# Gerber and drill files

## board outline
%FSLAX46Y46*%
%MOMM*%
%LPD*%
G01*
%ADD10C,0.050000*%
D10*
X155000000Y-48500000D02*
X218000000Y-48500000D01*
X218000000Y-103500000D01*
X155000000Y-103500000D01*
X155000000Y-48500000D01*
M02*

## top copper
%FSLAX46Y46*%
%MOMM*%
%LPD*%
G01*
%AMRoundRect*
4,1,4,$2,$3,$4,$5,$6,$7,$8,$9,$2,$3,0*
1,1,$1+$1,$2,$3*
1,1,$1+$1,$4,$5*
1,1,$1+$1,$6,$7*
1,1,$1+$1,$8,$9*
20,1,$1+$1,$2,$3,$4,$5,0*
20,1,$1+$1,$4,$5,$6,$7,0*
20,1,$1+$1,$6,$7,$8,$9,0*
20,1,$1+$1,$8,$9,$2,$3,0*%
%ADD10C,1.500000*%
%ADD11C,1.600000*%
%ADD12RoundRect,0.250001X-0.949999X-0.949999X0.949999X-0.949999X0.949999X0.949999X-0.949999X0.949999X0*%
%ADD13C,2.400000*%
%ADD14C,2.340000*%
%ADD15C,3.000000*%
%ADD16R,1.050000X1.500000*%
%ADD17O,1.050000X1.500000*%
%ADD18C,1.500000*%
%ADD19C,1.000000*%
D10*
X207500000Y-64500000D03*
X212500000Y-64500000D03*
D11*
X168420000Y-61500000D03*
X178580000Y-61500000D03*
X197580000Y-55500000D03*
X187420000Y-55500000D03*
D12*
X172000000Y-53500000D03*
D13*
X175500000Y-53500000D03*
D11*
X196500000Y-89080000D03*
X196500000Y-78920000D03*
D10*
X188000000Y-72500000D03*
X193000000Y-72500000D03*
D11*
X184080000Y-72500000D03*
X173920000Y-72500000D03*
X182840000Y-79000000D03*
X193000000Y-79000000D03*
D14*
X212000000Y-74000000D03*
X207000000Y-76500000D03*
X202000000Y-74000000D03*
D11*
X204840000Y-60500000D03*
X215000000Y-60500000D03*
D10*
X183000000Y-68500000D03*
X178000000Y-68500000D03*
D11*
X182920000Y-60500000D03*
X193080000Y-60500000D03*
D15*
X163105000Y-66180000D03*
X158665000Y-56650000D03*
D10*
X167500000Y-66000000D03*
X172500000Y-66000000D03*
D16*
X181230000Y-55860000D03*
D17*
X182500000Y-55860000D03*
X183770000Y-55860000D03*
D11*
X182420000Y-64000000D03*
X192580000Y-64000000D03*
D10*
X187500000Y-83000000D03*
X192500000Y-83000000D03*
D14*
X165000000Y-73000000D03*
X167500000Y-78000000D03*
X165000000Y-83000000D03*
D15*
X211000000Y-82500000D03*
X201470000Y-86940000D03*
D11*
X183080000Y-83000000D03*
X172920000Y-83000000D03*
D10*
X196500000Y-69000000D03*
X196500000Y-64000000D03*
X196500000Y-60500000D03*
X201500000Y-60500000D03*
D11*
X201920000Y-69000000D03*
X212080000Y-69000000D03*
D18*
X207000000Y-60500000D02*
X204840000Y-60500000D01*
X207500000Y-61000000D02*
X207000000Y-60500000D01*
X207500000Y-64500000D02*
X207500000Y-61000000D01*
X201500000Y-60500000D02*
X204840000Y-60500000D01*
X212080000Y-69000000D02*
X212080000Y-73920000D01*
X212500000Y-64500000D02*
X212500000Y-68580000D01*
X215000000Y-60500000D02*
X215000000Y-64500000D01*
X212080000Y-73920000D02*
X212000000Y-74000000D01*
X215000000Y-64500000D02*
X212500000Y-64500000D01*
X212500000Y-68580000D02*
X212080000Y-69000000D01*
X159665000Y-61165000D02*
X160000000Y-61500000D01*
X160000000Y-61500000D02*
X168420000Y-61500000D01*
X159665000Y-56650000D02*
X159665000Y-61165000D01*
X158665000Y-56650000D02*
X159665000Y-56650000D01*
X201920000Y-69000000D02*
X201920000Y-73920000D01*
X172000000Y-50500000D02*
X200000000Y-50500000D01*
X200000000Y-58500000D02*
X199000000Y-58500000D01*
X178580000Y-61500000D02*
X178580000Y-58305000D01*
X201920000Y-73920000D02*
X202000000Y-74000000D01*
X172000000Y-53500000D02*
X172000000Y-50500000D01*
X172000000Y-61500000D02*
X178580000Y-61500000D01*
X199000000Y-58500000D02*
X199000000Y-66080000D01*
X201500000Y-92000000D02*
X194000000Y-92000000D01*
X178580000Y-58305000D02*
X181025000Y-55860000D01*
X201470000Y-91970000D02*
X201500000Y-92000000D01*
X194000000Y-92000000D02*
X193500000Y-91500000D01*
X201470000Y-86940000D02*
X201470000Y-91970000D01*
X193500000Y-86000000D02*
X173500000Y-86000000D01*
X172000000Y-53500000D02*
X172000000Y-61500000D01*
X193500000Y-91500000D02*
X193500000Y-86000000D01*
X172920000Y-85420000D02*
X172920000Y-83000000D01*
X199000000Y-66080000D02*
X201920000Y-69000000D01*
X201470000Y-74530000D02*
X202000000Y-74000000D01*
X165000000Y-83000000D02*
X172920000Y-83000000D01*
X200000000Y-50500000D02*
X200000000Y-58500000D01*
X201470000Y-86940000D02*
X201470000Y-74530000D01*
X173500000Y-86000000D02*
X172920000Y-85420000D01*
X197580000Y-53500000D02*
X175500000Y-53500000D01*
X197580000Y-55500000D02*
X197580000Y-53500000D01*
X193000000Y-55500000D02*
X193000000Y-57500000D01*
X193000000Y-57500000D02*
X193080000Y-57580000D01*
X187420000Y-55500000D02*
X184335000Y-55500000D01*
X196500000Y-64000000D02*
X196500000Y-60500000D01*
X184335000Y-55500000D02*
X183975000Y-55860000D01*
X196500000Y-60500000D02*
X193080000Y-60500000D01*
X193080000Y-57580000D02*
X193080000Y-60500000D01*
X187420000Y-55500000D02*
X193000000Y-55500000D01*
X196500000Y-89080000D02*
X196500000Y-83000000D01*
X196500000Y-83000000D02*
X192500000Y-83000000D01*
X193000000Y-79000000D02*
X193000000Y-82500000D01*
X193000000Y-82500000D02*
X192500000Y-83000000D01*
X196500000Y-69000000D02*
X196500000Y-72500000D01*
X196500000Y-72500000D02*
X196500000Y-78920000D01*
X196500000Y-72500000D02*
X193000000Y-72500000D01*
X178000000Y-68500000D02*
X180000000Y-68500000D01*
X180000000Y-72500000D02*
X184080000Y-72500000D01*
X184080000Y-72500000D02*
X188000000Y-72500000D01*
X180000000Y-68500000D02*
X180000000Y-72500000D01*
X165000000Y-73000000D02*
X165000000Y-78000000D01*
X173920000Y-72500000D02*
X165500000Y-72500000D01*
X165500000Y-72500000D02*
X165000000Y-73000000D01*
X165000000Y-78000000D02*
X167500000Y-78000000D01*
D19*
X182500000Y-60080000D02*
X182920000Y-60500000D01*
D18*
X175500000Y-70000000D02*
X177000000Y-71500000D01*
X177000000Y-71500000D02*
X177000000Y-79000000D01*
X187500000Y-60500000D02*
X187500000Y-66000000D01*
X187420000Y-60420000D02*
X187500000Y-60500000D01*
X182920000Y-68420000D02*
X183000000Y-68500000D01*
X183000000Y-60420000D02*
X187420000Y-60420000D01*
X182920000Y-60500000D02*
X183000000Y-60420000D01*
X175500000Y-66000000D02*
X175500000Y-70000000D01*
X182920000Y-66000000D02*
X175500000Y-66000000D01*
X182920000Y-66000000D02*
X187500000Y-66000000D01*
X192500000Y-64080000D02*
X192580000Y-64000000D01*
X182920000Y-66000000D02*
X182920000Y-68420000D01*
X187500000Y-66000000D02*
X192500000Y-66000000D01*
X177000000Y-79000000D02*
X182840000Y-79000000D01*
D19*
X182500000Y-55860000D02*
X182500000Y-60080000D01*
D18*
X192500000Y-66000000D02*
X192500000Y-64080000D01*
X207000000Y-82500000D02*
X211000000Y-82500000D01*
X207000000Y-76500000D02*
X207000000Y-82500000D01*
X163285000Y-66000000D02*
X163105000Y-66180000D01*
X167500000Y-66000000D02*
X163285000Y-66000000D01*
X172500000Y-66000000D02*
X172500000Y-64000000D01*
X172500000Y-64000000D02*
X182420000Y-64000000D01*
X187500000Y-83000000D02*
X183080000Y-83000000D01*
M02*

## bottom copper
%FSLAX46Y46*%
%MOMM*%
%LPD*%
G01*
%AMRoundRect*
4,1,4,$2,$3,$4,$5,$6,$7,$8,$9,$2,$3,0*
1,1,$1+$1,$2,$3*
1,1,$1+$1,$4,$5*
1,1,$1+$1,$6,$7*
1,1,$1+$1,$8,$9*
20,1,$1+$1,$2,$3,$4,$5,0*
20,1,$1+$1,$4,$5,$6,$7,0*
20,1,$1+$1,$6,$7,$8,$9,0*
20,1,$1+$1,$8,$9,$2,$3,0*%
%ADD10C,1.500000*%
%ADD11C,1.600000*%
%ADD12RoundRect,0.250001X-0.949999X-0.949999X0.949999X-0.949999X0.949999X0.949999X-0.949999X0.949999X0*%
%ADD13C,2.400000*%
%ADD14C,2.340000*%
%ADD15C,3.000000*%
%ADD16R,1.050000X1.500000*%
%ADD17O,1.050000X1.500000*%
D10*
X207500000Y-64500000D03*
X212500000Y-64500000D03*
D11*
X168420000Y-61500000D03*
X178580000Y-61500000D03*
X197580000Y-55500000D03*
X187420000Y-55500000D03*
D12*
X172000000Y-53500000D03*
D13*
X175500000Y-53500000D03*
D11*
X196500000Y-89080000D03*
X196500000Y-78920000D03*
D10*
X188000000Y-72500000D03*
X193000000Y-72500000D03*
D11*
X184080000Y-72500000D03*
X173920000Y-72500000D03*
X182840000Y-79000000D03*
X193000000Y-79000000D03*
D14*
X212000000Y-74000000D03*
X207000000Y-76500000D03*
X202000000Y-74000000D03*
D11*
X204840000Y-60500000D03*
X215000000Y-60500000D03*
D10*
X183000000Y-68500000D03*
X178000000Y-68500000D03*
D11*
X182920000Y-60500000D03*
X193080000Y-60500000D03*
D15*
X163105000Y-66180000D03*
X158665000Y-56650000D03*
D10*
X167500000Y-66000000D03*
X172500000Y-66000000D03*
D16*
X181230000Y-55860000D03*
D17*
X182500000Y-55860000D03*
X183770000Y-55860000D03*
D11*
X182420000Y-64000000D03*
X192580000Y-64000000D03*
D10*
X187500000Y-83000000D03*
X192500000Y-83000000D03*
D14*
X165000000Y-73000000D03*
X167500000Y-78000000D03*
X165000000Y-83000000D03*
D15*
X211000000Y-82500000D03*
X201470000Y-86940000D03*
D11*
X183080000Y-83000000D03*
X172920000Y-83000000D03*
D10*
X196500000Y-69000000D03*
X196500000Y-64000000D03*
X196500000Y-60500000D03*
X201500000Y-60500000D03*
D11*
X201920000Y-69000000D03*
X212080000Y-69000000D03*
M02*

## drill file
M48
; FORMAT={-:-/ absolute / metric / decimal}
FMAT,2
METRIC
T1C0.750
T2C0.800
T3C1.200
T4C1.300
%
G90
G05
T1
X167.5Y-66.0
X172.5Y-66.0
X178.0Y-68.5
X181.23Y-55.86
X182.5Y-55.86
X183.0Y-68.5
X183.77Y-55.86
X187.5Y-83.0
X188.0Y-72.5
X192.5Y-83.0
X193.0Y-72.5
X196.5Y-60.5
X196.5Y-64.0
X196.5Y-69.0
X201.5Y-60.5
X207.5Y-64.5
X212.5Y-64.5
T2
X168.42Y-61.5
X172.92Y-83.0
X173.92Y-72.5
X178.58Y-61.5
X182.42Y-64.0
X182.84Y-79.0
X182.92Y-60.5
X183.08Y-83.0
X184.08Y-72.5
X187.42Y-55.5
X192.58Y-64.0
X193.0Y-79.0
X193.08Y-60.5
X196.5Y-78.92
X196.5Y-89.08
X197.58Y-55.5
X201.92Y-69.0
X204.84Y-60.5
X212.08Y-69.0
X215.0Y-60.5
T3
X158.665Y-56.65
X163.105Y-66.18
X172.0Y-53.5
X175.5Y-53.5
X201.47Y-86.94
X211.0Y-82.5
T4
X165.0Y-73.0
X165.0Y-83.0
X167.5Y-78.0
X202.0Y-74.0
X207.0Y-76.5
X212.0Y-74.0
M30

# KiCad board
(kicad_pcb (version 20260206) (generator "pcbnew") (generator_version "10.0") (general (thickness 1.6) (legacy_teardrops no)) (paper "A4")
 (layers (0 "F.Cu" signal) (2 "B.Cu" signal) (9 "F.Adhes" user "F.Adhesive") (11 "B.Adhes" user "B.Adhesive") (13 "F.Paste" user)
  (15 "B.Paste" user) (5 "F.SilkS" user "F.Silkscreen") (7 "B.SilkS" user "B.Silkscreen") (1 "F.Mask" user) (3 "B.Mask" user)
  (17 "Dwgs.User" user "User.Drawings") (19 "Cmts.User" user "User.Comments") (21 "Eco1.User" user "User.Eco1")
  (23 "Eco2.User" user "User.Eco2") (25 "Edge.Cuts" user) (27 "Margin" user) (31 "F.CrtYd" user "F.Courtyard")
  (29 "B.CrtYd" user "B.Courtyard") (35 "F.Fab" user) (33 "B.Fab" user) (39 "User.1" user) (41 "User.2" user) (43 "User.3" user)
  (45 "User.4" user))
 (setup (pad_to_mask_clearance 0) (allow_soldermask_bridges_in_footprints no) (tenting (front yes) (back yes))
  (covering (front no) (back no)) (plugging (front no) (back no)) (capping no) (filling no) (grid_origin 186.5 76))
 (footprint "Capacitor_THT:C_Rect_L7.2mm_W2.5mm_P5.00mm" (layer "F.Cu") (at 207.5 64.5)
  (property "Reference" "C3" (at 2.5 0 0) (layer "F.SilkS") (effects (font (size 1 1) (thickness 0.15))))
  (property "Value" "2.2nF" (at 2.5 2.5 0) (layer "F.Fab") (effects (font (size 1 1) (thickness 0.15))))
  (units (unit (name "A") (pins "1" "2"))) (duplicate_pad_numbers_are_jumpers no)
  (pad "1" thru_hole circle (at 0 0) (size 1.5 1.5) (drill 0.75) (layers "*.Cu" "*.Mask") (remove_unused_layers no) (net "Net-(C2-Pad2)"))
  (pad "2" thru_hole circle (at 5 0) (size 1.5 1.5) (drill 0.75) (layers "*.Cu" "*.Mask") (remove_unused_layers no) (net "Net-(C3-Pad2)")))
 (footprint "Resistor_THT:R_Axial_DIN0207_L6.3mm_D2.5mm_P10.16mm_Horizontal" (layer "F.Cu") (at 168.42 61.5)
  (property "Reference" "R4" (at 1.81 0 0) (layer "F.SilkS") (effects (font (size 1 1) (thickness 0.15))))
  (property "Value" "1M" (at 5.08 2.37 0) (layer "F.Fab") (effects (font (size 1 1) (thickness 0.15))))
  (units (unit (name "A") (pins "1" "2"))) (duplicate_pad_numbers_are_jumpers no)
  (pad "1" thru_hole circle (at 0 0) (size 1.6 1.6) (drill 0.8) (layers "*.Cu" "*.Mask") (remove_unused_layers no) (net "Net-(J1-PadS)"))
  (pad "2" thru_hole circle (at 10.16 0) (size 1.6 1.6) (drill 0.8) (layers "*.Cu" "*.Mask") (remove_unused_layers no) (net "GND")))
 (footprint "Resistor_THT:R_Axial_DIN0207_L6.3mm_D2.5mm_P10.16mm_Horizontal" (layer "F.Cu") (at 197.58 55.5 180)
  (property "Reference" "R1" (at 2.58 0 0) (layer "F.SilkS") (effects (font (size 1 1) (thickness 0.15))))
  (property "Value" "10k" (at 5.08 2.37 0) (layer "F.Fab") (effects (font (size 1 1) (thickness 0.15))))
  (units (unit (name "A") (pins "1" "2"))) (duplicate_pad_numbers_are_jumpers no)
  (pad "1" thru_hole circle (at 0 0 180) (size 1.6 1.6) (drill 0.8) (layers "*.Cu" "*.Mask") (remove_unused_layers no) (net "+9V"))
  (pad "2" thru_hole circle (at 10.16 0 180) (size 1.6 1.6) (drill 0.8) (layers "*.Cu" "*.Mask") (remove_unused_layers no)
   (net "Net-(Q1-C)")))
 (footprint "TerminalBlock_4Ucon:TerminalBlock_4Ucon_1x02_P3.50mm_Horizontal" (layer "F.Cu") (at 172 53.5)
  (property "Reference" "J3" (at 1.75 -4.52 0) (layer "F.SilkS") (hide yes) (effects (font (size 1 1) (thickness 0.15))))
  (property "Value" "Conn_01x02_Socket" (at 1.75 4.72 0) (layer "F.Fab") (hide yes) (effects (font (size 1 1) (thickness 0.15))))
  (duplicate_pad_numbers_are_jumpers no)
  (pad "1" thru_hole roundrect (at 0 0) (size 2.4 2.4) (drill 1.2) (layers "*.Cu" "*.Mask") (remove_unused_layers no)
   (roundrect_rratio 0.104167) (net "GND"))
  (pad "2" thru_hole circle (at 3.5 0) (size 2.4 2.4) (drill 1.2) (layers "*.Cu" "*.Mask") (remove_unused_layers no) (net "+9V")))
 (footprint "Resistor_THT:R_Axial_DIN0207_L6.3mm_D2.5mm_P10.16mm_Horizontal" (layer "F.Cu") (at 196.5 89.08 90)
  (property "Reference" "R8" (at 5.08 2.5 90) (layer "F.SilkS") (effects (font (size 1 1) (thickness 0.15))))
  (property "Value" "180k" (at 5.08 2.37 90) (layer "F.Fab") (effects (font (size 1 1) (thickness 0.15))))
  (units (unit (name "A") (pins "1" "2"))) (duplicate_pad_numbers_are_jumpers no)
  (pad "1" thru_hole circle (at 0 0 90) (size 1.6 1.6) (drill 0.8) (layers "*.Cu" "*.Mask") (remove_unused_layers no) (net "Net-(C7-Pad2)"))
  (pad "2" thru_hole circle (at 10.16 0 90) (size 1.6 1.6) (drill 0.8) (layers "*.Cu" "*.Mask") (remove_unused_layers no)
   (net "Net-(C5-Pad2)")))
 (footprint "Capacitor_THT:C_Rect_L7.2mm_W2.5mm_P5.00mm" (layer "F.Cu") (at 188 72.5)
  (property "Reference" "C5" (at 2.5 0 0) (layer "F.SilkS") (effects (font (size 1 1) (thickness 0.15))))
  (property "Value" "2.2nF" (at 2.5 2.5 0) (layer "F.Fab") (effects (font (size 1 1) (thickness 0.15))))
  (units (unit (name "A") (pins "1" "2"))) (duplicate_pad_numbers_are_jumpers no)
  (pad "1" thru_hole circle (at 0 0) (size 1.5 1.5) (drill 0.75) (layers "*.Cu" "*.Mask") (remove_unused_layers no) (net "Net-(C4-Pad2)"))
  (pad "2" thru_hole circle (at 5 0) (size 1.5 1.5) (drill 0.75) (layers "*.Cu" "*.Mask") (remove_unused_layers no) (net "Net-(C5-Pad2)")))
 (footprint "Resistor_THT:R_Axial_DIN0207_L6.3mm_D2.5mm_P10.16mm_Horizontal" (layer "F.Cu") (at 184.08 72.5 180)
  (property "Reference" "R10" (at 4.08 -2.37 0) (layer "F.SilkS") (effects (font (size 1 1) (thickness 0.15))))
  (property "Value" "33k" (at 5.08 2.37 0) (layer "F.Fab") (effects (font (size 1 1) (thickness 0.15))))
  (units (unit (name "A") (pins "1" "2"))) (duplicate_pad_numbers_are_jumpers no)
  (pad "1" thru_hole circle (at 0 0 180) (size 1.6 1.6) (drill 0.8) (layers "*.Cu" "*.Mask") (remove_unused_layers no) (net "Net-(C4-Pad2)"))
  (pad "2" thru_hole circle (at 10.16 0 180) (size 1.6 1.6) (drill 0.8) (layers "*.Cu" "*.Mask") (remove_unused_layers no)
   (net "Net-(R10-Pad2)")))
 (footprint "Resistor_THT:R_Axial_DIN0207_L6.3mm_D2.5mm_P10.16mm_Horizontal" (layer "F.Cu") (at 182.84 79)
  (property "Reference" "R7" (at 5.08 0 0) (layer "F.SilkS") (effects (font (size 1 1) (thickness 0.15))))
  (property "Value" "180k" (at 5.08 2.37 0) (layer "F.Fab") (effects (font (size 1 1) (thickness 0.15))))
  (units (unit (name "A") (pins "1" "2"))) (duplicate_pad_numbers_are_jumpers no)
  (pad "1" thru_hole circle (at 0 0) (size 1.6 1.6) (drill 0.8) (layers "*.Cu" "*.Mask") (remove_unused_layers no) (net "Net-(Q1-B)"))
  (pad "2" thru_hole circle (at 10.16 0) (size 1.6 1.6) (drill 0.8) (layers "*.Cu" "*.Mask") (remove_unused_layers no) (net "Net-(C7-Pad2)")))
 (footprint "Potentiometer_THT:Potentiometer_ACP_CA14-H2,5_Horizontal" (layer "F.Cu") (at 212 74 -90)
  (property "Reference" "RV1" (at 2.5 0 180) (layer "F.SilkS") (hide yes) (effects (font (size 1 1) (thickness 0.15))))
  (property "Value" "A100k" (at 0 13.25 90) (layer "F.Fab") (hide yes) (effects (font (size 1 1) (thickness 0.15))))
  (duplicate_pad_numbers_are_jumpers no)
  (pad "1" thru_hole circle (at 0 0 270) (size 2.34 2.34) (drill 1.3) (layers "*.Cu" "*.Mask") (remove_unused_layers no)
   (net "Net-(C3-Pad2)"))
  (pad "2" thru_hole circle (at 2.5 5 270) (size 2.34 2.34) (drill 1.3) (layers "*.Cu" "*.Mask") (remove_unused_layers no)
   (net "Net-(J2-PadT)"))
  (pad "3" thru_hole circle (at 0 10 270) (size 2.34 2.34) (drill 1.3) (layers "*.Cu" "*.Mask") (remove_unused_layers no) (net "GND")))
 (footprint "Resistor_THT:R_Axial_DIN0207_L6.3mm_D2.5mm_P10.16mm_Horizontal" (layer "F.Cu") (at 204.84 60.5)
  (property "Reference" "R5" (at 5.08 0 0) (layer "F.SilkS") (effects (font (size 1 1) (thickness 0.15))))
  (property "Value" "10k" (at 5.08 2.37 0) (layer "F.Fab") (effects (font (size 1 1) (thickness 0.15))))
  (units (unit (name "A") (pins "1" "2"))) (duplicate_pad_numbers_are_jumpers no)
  (pad "1" thru_hole circle (at 0 0) (size 1.6 1.6) (drill 0.8) (layers "*.Cu" "*.Mask") (remove_unused_layers no) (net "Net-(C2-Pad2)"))
  (pad "2" thru_hole circle (at 10.16 0) (size 1.6 1.6) (drill 0.8) (layers "*.Cu" "*.Mask") (remove_unused_layers no) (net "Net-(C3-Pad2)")))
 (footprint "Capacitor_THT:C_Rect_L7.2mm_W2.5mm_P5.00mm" (layer "F.Cu") (at 183 68.5 180)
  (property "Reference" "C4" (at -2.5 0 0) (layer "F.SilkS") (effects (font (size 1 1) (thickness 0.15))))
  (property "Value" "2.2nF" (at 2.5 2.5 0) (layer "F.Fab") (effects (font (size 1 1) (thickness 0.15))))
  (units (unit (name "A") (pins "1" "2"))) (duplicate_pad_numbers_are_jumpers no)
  (pad "1" thru_hole circle (at 0 0 180) (size 1.5 1.5) (drill 0.75) (layers "*.Cu" "*.Mask") (remove_unused_layers no) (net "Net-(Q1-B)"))
  (pad "2" thru_hole circle (at 5 0 180) (size 1.5 1.5) (drill 0.75) (layers "*.Cu" "*.Mask") (remove_unused_layers no)
   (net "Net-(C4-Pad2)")))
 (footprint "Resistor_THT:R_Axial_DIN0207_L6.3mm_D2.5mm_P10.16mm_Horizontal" (layer "F.Cu") (at 182.92 60.5)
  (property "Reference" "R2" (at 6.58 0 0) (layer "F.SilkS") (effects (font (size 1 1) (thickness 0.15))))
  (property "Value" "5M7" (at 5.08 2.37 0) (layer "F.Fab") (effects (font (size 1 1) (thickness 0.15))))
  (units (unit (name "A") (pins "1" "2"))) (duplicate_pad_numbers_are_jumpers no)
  (pad "1" thru_hole circle (at 0 0) (size 1.6 1.6) (drill 0.8) (layers "*.Cu" "*.Mask") (remove_unused_layers no) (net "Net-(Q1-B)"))
  (pad "2" thru_hole circle (at 10.16 0) (size 1.6 1.6) (drill 0.8) (layers "*.Cu" "*.Mask") (remove_unused_layers no) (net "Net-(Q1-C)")))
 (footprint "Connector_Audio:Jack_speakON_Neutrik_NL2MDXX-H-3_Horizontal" (layer "F.Cu") (at 163.105 66.18 180)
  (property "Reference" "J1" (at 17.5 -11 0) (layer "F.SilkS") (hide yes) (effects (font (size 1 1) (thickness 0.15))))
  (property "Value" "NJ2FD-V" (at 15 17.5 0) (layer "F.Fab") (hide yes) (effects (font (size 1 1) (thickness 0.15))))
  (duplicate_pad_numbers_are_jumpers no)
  (pad "1+" thru_hole circle (at 0 0 180) (size 3 3) (drill 1.2) (layers "*.Cu" "*.Mask") (remove_unused_layers no) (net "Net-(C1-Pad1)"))
  (pad "1-" thru_hole circle (at 4.44 9.53 180) (size 3 3) (drill 1.2) (layers "*.Cu" "*.Mask") (remove_unused_layers no)
   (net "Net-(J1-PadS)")))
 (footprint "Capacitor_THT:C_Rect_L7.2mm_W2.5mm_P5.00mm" (layer "F.Cu") (at 167.5 66)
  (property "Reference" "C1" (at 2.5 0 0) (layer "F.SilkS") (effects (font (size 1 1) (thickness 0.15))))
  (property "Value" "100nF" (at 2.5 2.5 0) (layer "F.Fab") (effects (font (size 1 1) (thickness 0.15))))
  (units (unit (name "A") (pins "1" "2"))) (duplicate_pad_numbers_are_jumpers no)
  (pad "1" thru_hole circle (at 0 0) (size 1.5 1.5) (drill 0.75) (layers "*.Cu" "*.Mask") (remove_unused_layers no) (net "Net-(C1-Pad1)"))
  (pad "2" thru_hole circle (at 5 0) (size 1.5 1.5) (drill 0.75) (layers "*.Cu" "*.Mask") (remove_unused_layers no) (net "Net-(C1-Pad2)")))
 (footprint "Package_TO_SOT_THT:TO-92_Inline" (layer "F.Cu") (at 181.23 55.86)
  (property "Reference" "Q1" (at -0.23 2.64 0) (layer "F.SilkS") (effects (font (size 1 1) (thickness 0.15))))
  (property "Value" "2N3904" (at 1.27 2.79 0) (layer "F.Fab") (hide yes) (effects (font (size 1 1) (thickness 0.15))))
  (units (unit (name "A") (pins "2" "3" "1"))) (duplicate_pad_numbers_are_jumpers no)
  (pad "1" thru_hole rect (at 0 0) (size 1.05 1.5) (drill 0.75) (layers "*.Cu" "*.Mask") (remove_unused_layers no) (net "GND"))
  (pad "2" thru_hole oval (at 1.27 0) (size 1.05 1.5) (drill 0.75) (layers "*.Cu" "*.Mask") (remove_unused_layers no) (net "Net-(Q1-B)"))
  (pad "3" thru_hole oval (at 2.54 0) (size 1.05 1.5) (drill 0.75) (layers "*.Cu" "*.Mask") (remove_unused_layers no) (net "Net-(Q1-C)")))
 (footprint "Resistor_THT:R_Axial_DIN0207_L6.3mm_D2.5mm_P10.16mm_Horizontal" (layer "F.Cu") (at 182.42 64)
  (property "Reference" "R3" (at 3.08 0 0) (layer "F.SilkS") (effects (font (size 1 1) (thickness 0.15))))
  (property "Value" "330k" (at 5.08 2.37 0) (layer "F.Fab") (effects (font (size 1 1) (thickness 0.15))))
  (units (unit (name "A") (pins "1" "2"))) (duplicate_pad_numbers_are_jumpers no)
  (pad "1" thru_hole circle (at 0 0) (size 1.6 1.6) (drill 0.8) (layers "*.Cu" "*.Mask") (remove_unused_layers no) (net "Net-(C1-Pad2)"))
  (pad "2" thru_hole circle (at 10.16 0) (size 1.6 1.6) (drill 0.8) (layers "*.Cu" "*.Mask") (remove_unused_layers no) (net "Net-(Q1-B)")))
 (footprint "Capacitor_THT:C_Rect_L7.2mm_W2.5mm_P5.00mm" (layer "F.Cu") (at 187.5 83)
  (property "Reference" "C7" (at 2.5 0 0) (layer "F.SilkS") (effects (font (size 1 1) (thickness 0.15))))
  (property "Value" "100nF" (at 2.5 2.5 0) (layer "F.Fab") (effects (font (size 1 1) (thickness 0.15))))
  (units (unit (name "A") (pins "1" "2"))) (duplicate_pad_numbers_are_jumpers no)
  (pad "1" thru_hole circle (at 0 0) (size 1.5 1.5) (drill 0.75) (layers "*.Cu" "*.Mask") (remove_unused_layers no) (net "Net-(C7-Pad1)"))
  (pad "2" thru_hole circle (at 5 0) (size 1.5 1.5) (drill 0.75) (layers "*.Cu" "*.Mask") (remove_unused_layers no) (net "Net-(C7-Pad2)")))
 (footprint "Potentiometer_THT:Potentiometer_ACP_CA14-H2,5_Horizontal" (layer "F.Cu") (at 165 73)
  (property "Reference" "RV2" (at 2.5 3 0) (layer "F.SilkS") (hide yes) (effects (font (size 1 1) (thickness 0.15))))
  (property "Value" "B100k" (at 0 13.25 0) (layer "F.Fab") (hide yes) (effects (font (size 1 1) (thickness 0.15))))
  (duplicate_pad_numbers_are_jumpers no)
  (pad "1" thru_hole circle (at 0 0) (size 2.34 2.34) (drill 1.3) (layers "*.Cu" "*.Mask") (remove_unused_layers no) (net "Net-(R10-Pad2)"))
  (pad "2" thru_hole circle (at 2.5 5) (size 2.34 2.34) (drill 1.3) (layers "*.Cu" "*.Mask") (remove_unused_layers no)
   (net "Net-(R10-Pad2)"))
  (pad "3" thru_hole circle (at 0 10) (size 2.34 2.34) (drill 1.3) (layers "*.Cu" "*.Mask") (remove_unused_layers no) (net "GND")))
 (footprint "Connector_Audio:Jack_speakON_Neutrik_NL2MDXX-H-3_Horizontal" (layer "F.Cu") (at 211 82.5 -90)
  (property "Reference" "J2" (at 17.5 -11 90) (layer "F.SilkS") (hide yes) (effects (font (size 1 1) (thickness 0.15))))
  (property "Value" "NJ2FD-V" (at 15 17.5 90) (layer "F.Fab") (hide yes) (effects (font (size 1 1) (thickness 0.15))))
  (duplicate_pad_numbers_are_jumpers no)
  (pad "1+" thru_hole circle (at 0 0 270) (size 3 3) (drill 1.2) (layers "*.Cu" "*.Mask") (remove_unused_layers no) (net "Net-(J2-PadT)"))
  (pad "1-" thru_hole circle (at 4.44 9.53 270) (size 3 3) (drill 1.2) (layers "*.Cu" "*.Mask") (remove_unused_layers no) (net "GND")))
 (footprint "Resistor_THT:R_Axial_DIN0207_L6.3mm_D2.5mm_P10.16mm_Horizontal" (layer "F.Cu") (at 183.08 83 180)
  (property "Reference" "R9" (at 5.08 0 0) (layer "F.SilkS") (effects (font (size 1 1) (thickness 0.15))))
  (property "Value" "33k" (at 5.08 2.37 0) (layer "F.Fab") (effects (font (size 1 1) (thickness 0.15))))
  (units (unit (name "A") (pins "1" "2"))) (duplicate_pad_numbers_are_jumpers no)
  (pad "1" thru_hole circle (at 0 0 180) (size 1.6 1.6) (drill 0.8) (layers "*.Cu" "*.Mask") (remove_unused_layers no) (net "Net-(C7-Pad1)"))
  (pad "2" thru_hole circle (at 10.16 0 180) (size 1.6 1.6) (drill 0.8) (layers "*.Cu" "*.Mask") (remove_unused_layers no) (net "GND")))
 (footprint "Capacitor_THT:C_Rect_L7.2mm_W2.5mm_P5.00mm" (layer "F.Cu") (at 196.5 69 90)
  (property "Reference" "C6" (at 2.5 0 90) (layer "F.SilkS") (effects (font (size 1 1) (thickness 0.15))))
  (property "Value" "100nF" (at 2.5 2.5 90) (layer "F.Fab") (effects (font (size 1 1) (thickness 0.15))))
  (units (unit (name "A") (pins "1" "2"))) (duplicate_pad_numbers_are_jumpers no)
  (pad "1" thru_hole circle (at 0 0 90) (size 1.5 1.5) (drill 0.75) (layers "*.Cu" "*.Mask") (remove_unused_layers no) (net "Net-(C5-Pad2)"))
  (pad "2" thru_hole circle (at 5 0 90) (size 1.5 1.5) (drill 0.75) (layers "*.Cu" "*.Mask") (remove_unused_layers no) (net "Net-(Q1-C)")))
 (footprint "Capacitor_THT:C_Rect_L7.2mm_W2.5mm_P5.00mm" (layer "F.Cu") (at 196.5 60.5)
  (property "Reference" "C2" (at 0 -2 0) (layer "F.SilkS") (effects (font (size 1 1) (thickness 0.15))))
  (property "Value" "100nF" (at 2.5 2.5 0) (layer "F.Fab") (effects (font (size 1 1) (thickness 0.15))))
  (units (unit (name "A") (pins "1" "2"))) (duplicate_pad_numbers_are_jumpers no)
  (pad "1" thru_hole circle (at 0 0) (size 1.5 1.5) (drill 0.75) (layers "*.Cu" "*.Mask") (remove_unused_layers no) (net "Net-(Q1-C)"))
  (pad "2" thru_hole circle (at 5 0) (size 1.5 1.5) (drill 0.75) (layers "*.Cu" "*.Mask") (remove_unused_layers no) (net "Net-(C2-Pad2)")))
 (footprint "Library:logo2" (layer "F.Cu") (at 186.500278 97.619189)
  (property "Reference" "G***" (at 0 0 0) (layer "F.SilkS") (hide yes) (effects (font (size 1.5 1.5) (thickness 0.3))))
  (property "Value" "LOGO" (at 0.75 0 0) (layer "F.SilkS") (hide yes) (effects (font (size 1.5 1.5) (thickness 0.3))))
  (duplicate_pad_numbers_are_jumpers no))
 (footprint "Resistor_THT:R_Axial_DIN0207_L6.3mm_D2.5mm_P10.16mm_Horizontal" (layer "F.Cu") (at 201.92 69)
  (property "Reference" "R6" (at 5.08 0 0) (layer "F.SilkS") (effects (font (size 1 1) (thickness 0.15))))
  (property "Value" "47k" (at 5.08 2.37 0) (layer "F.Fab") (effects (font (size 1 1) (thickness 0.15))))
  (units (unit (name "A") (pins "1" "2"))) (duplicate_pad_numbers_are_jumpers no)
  (pad "1" thru_hole circle (at 0 0) (size 1.6 1.6) (drill 0.8) (layers "*.Cu" "*.Mask") (remove_unused_layers no) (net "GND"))
  (pad "2" thru_hole circle (at 10.16 0) (size 1.6 1.6) (drill 0.8) (layers "*.Cu" "*.Mask") (remove_unused_layers no) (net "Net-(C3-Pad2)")))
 (gr_rect (start 155 48.5) (end 218 103.5) (stroke (width 0.05) (type default)) (fill no) (layer "Edge.Cuts"))
 (segment (start 207 60.5) (end 204.84 60.5) (width 1.5) (layer "F.Cu") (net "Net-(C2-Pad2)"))
 (segment (start 207.5 61) (end 207 60.5) (width 1.5) (layer "F.Cu") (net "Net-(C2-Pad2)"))
 (segment (start 207.5 64.5) (end 207.5 61) (width 1.5) (layer "F.Cu") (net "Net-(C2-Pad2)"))
 (segment (start 201.5 60.5) (end 204.84 60.5) (width 1.5) (layer "F.Cu") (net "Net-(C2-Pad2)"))
 (segment (start 212.08 69) (end 212.08 73.92) (width 1.5) (layer "F.Cu") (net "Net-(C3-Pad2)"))
 (segment (start 212.5 64.5) (end 212.5 68.58) (width 1.5) (layer "F.Cu") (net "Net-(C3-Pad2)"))
 (segment (start 215 60.5) (end 215 64.5) (width 1.5) (layer "F.Cu") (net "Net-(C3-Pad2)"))
 (segment (start 212.08 73.92) (end 212 74) (width 1.5) (layer "F.Cu") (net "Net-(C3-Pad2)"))
 (segment (start 215 64.5) (end 212.5 64.5) (width 1.5) (layer "F.Cu") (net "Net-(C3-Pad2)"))
 (segment (start 212.5 68.58) (end 212.08 69) (width 1.5) (layer "F.Cu") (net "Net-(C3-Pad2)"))
 (segment (start 159.665 61.165) (end 160 61.5) (width 1.5) (layer "F.Cu") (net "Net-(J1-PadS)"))
 (segment (start 160 61.5) (end 168.42 61.5) (width 1.5) (layer "F.Cu") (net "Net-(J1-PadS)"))
 (segment (start 159.665 56.65) (end 159.665 61.165) (width 1.5) (layer "F.Cu") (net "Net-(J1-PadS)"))
 (segment (start 158.665 56.65) (end 159.665 56.65) (width 1.5) (layer "F.Cu") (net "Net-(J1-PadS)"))
 (segment (start 201.92 69) (end 201.92 73.92) (width 1.5) (layer "F.Cu") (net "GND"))
 (segment (start 172 50.5) (end 200 50.5) (width 1.5) (layer "F.Cu") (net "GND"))
 (segment (start 200 58.5) (end 199 58.5) (width 1.5) (layer "F.Cu") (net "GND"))
 (segment (start 178.58 61.5) (end 178.58 58.305) (width 1.5) (layer "F.Cu") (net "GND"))
 (segment (start 201.92 73.92) (end 202 74) (width 1.5) (layer "F.Cu") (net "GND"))
 (segment (start 172 53.5) (end 172 50.5) (width 1.5) (layer "F.Cu") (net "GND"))
 (segment (start 172 61.5) (end 178.58 61.5) (width 1.5) (layer "F.Cu") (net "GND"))
 (segment (start 199 58.5) (end 199 66.08) (width 1.5) (layer "F.Cu") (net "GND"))
 (segment (start 201.5 92) (end 194 92) (width 1.5) (layer "F.Cu") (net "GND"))
 (segment (start 178.58 58.305) (end 181.025 55.86) (width 1.5) (layer "F.Cu") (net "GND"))
 (segment (start 201.47 91.97) (end 201.5 92) (width 1.5) (layer "F.Cu") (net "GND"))
 (segment (start 194 92) (end 193.5 91.5) (width 1.5) (layer "F.Cu") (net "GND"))
 (segment (start 201.47 86.94) (end 201.47 91.97) (width 1.5) (layer "F.Cu") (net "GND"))
 (segment (start 193.5 86) (end 173.5 86) (width 1.5) (layer "F.Cu") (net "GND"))
 (segment (start 172 53.5) (end 172 61.5) (width 1.5) (layer "F.Cu") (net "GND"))
 (segment (start 193.5 91.5) (end 193.5 86) (width 1.5) (layer "F.Cu") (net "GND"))
 (segment (start 172.92 85.42) (end 172.92 83) (width 1.5) (layer "F.Cu") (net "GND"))
 (segment (start 199 66.08) (end 201.92 69) (width 1.5) (layer "F.Cu") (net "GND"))
 (segment (start 201.47 74.53) (end 202 74) (width 1.5) (layer "F.Cu") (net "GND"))
 (segment (start 165 83) (end 172.92 83) (width 1.5) (layer "F.Cu") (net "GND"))
 (segment (start 200 50.5) (end 200 58.5) (width 1.5) (layer "F.Cu") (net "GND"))
 (segment (start 201.47 86.94) (end 201.47 74.53) (width 1.5) (layer "F.Cu") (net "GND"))
 (segment (start 173.5 86) (end 172.92 85.42) (width 1.5) (layer "F.Cu") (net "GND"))
 (segment (start 197.58 53.5) (end 175.5 53.5) (width 1.5) (layer "F.Cu") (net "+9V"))
 (segment (start 197.58 55.5) (end 197.58 53.5) (width 1.5) (layer "F.Cu") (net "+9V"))
 (segment (start 193 55.5) (end 193 57.5) (width 1.5) (layer "F.Cu") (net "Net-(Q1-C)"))
 (segment (start 193 57.5) (end 193.08 57.58) (width 1.5) (layer "F.Cu") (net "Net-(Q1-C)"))
 (segment (start 187.42 55.5) (end 184.335 55.5) (width 1.5) (layer "F.Cu") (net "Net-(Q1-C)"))
 (segment (start 196.5 64) (end 196.5 60.5) (width 1.5) (layer "F.Cu") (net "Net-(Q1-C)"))
 (segment (start 184.335 55.5) (end 183.975 55.86) (width 1.5) (layer "F.Cu") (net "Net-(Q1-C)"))
 (segment (start 196.5 60.5) (end 193.08 60.5) (width 1.5) (layer "F.Cu") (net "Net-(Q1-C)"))
 (segment (start 193.08 57.58) (end 193.08 60.5) (width 1.5) (layer "F.Cu") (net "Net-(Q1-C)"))
 (segment (start 187.42 55.5) (end 193 55.5) (width 1.5) (layer "F.Cu") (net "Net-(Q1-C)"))
 (segment (start 196.5 89.08) (end 196.5 83) (width 1.5) (layer "F.Cu") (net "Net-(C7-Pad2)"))
 (segment (start 196.5 83) (end 192.5 83) (width 1.5) (layer "F.Cu") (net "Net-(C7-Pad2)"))
 (segment (start 193 79) (end 193 82.5) (width 1.5) (layer "F.Cu") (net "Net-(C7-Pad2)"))
 (segment (start 193 82.5) (end 192.5 83) (width 1.5) (layer "F.Cu") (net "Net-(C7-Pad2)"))
 (segment (start 196.5 69) (end 196.5 72.5) (width 1.5) (layer "F.Cu") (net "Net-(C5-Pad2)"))
 (segment (start 196.5 72.5) (end 196.5 78.92) (width 1.5) (layer "F.Cu") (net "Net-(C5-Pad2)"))
 (segment (start 196.5 72.5) (end 193 72.5) (width 1.5) (layer "F.Cu") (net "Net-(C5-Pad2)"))
 (segment (start 178 68.5) (end 180 68.5) (width 1.5) (layer "F.Cu") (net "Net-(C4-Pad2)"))
 (segment (start 180 72.5) (end 184.08 72.5) (width 1.5) (layer "F.Cu") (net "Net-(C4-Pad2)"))
 (segment (start 184.08 72.5) (end 188 72.5) (width 1.5) (layer "F.Cu") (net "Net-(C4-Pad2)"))
 (segment (start 180 68.5) (end 180 72.5) (width 1.5) (layer "F.Cu") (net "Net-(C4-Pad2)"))
 (segment (start 165 73) (end 165 78) (width 1.5) (layer "F.Cu") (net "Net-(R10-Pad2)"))
 (segment (start 173.92 72.5) (end 165.5 72.5) (width 1.5) (layer "F.Cu") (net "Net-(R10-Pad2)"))
 (segment (start 165.5 72.5) (end 165 73) (width 1.5) (layer "F.Cu") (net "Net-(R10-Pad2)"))
 (segment (start 165 78) (end 167.5 78) (width 1.5) (layer "F.Cu") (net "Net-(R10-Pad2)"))
 (segment (start 182.5 60.08) (end 182.92 60.5) (width 1) (layer "F.Cu") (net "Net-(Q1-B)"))
 (segment (start 175.5 70) (end 177 71.5) (width 1.5) (layer "F.Cu") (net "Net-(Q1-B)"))
 (segment (start 177 71.5) (end 177 79) (width 1.5) (layer "F.Cu") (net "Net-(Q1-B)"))
 (segment (start 187.5 60.5) (end 187.5 66) (width 1.5) (layer "F.Cu") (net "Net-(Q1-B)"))
 (segment (start 187.42 60.42) (end 187.5 60.5) (width 1.5) (layer "F.Cu") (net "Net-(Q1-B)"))
 (segment (start 182.92 68.42) (end 183 68.5) (width 1.5) (layer "F.Cu") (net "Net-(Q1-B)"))
 (segment (start 183 60.42) (end 187.42 60.42) (width 1.5) (layer "F.Cu") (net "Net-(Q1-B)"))
 (segment (start 182.92 60.5) (end 183 60.42) (width 1.5) (layer "F.Cu") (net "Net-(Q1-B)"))
 (segment (start 175.5 66) (end 175.5 70) (width 1.5) (layer "F.Cu") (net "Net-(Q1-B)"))
 (segment (start 182.92 66) (end 175.5 66) (width 1.5) (layer "F.Cu") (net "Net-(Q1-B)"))
 (segment (start 182.92 66) (end 187.5 66) (width 1.5) (layer "F.Cu") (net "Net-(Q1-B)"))
 (segment (start 192.5 64.08) (end 192.58 64) (width 1.5) (layer "F.Cu") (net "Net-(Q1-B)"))
 (segment (start 182.92 66) (end 182.92 68.42) (width 1.5) (layer "F.Cu") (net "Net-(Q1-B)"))
 (segment (start 187.5 66) (end 192.5 66) (width 1.5) (layer "F.Cu") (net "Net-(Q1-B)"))
 (segment (start 177 79) (end 182.84 79) (width 1.5) (layer "F.Cu") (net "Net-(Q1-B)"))
 (segment (start 182.5 55.86) (end 182.5 60.08) (width 1) (layer "F.Cu") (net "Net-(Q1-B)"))
 (segment (start 192.5 66) (end 192.5 64.08) (width 1.5) (layer "F.Cu") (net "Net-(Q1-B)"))
 (segment (start 207 82.5) (end 211 82.5) (width 1.5) (layer "F.Cu") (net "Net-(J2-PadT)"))
 (segment (start 207 76.5) (end 207 82.5) (width 1.5) (layer "F.Cu") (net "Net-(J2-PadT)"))
 (segment (start 163.285 66) (end 163.105 66.18) (width 1.5) (layer "F.Cu") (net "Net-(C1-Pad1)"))
 (segment (start 167.5 66) (end 163.285 66) (width 1.5) (layer "F.Cu") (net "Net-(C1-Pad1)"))
 (segment (start 172.5 66) (end 172.5 64) (width 1.5) (layer "F.Cu") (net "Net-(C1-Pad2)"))
 (segment (start 172.5 64) (end 182.42 64) (width 1.5) (layer "F.Cu") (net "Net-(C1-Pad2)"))
 (segment (start 187.5 83) (end 183.08 83) (width 1.5) (layer "F.Cu") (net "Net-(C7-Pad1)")))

